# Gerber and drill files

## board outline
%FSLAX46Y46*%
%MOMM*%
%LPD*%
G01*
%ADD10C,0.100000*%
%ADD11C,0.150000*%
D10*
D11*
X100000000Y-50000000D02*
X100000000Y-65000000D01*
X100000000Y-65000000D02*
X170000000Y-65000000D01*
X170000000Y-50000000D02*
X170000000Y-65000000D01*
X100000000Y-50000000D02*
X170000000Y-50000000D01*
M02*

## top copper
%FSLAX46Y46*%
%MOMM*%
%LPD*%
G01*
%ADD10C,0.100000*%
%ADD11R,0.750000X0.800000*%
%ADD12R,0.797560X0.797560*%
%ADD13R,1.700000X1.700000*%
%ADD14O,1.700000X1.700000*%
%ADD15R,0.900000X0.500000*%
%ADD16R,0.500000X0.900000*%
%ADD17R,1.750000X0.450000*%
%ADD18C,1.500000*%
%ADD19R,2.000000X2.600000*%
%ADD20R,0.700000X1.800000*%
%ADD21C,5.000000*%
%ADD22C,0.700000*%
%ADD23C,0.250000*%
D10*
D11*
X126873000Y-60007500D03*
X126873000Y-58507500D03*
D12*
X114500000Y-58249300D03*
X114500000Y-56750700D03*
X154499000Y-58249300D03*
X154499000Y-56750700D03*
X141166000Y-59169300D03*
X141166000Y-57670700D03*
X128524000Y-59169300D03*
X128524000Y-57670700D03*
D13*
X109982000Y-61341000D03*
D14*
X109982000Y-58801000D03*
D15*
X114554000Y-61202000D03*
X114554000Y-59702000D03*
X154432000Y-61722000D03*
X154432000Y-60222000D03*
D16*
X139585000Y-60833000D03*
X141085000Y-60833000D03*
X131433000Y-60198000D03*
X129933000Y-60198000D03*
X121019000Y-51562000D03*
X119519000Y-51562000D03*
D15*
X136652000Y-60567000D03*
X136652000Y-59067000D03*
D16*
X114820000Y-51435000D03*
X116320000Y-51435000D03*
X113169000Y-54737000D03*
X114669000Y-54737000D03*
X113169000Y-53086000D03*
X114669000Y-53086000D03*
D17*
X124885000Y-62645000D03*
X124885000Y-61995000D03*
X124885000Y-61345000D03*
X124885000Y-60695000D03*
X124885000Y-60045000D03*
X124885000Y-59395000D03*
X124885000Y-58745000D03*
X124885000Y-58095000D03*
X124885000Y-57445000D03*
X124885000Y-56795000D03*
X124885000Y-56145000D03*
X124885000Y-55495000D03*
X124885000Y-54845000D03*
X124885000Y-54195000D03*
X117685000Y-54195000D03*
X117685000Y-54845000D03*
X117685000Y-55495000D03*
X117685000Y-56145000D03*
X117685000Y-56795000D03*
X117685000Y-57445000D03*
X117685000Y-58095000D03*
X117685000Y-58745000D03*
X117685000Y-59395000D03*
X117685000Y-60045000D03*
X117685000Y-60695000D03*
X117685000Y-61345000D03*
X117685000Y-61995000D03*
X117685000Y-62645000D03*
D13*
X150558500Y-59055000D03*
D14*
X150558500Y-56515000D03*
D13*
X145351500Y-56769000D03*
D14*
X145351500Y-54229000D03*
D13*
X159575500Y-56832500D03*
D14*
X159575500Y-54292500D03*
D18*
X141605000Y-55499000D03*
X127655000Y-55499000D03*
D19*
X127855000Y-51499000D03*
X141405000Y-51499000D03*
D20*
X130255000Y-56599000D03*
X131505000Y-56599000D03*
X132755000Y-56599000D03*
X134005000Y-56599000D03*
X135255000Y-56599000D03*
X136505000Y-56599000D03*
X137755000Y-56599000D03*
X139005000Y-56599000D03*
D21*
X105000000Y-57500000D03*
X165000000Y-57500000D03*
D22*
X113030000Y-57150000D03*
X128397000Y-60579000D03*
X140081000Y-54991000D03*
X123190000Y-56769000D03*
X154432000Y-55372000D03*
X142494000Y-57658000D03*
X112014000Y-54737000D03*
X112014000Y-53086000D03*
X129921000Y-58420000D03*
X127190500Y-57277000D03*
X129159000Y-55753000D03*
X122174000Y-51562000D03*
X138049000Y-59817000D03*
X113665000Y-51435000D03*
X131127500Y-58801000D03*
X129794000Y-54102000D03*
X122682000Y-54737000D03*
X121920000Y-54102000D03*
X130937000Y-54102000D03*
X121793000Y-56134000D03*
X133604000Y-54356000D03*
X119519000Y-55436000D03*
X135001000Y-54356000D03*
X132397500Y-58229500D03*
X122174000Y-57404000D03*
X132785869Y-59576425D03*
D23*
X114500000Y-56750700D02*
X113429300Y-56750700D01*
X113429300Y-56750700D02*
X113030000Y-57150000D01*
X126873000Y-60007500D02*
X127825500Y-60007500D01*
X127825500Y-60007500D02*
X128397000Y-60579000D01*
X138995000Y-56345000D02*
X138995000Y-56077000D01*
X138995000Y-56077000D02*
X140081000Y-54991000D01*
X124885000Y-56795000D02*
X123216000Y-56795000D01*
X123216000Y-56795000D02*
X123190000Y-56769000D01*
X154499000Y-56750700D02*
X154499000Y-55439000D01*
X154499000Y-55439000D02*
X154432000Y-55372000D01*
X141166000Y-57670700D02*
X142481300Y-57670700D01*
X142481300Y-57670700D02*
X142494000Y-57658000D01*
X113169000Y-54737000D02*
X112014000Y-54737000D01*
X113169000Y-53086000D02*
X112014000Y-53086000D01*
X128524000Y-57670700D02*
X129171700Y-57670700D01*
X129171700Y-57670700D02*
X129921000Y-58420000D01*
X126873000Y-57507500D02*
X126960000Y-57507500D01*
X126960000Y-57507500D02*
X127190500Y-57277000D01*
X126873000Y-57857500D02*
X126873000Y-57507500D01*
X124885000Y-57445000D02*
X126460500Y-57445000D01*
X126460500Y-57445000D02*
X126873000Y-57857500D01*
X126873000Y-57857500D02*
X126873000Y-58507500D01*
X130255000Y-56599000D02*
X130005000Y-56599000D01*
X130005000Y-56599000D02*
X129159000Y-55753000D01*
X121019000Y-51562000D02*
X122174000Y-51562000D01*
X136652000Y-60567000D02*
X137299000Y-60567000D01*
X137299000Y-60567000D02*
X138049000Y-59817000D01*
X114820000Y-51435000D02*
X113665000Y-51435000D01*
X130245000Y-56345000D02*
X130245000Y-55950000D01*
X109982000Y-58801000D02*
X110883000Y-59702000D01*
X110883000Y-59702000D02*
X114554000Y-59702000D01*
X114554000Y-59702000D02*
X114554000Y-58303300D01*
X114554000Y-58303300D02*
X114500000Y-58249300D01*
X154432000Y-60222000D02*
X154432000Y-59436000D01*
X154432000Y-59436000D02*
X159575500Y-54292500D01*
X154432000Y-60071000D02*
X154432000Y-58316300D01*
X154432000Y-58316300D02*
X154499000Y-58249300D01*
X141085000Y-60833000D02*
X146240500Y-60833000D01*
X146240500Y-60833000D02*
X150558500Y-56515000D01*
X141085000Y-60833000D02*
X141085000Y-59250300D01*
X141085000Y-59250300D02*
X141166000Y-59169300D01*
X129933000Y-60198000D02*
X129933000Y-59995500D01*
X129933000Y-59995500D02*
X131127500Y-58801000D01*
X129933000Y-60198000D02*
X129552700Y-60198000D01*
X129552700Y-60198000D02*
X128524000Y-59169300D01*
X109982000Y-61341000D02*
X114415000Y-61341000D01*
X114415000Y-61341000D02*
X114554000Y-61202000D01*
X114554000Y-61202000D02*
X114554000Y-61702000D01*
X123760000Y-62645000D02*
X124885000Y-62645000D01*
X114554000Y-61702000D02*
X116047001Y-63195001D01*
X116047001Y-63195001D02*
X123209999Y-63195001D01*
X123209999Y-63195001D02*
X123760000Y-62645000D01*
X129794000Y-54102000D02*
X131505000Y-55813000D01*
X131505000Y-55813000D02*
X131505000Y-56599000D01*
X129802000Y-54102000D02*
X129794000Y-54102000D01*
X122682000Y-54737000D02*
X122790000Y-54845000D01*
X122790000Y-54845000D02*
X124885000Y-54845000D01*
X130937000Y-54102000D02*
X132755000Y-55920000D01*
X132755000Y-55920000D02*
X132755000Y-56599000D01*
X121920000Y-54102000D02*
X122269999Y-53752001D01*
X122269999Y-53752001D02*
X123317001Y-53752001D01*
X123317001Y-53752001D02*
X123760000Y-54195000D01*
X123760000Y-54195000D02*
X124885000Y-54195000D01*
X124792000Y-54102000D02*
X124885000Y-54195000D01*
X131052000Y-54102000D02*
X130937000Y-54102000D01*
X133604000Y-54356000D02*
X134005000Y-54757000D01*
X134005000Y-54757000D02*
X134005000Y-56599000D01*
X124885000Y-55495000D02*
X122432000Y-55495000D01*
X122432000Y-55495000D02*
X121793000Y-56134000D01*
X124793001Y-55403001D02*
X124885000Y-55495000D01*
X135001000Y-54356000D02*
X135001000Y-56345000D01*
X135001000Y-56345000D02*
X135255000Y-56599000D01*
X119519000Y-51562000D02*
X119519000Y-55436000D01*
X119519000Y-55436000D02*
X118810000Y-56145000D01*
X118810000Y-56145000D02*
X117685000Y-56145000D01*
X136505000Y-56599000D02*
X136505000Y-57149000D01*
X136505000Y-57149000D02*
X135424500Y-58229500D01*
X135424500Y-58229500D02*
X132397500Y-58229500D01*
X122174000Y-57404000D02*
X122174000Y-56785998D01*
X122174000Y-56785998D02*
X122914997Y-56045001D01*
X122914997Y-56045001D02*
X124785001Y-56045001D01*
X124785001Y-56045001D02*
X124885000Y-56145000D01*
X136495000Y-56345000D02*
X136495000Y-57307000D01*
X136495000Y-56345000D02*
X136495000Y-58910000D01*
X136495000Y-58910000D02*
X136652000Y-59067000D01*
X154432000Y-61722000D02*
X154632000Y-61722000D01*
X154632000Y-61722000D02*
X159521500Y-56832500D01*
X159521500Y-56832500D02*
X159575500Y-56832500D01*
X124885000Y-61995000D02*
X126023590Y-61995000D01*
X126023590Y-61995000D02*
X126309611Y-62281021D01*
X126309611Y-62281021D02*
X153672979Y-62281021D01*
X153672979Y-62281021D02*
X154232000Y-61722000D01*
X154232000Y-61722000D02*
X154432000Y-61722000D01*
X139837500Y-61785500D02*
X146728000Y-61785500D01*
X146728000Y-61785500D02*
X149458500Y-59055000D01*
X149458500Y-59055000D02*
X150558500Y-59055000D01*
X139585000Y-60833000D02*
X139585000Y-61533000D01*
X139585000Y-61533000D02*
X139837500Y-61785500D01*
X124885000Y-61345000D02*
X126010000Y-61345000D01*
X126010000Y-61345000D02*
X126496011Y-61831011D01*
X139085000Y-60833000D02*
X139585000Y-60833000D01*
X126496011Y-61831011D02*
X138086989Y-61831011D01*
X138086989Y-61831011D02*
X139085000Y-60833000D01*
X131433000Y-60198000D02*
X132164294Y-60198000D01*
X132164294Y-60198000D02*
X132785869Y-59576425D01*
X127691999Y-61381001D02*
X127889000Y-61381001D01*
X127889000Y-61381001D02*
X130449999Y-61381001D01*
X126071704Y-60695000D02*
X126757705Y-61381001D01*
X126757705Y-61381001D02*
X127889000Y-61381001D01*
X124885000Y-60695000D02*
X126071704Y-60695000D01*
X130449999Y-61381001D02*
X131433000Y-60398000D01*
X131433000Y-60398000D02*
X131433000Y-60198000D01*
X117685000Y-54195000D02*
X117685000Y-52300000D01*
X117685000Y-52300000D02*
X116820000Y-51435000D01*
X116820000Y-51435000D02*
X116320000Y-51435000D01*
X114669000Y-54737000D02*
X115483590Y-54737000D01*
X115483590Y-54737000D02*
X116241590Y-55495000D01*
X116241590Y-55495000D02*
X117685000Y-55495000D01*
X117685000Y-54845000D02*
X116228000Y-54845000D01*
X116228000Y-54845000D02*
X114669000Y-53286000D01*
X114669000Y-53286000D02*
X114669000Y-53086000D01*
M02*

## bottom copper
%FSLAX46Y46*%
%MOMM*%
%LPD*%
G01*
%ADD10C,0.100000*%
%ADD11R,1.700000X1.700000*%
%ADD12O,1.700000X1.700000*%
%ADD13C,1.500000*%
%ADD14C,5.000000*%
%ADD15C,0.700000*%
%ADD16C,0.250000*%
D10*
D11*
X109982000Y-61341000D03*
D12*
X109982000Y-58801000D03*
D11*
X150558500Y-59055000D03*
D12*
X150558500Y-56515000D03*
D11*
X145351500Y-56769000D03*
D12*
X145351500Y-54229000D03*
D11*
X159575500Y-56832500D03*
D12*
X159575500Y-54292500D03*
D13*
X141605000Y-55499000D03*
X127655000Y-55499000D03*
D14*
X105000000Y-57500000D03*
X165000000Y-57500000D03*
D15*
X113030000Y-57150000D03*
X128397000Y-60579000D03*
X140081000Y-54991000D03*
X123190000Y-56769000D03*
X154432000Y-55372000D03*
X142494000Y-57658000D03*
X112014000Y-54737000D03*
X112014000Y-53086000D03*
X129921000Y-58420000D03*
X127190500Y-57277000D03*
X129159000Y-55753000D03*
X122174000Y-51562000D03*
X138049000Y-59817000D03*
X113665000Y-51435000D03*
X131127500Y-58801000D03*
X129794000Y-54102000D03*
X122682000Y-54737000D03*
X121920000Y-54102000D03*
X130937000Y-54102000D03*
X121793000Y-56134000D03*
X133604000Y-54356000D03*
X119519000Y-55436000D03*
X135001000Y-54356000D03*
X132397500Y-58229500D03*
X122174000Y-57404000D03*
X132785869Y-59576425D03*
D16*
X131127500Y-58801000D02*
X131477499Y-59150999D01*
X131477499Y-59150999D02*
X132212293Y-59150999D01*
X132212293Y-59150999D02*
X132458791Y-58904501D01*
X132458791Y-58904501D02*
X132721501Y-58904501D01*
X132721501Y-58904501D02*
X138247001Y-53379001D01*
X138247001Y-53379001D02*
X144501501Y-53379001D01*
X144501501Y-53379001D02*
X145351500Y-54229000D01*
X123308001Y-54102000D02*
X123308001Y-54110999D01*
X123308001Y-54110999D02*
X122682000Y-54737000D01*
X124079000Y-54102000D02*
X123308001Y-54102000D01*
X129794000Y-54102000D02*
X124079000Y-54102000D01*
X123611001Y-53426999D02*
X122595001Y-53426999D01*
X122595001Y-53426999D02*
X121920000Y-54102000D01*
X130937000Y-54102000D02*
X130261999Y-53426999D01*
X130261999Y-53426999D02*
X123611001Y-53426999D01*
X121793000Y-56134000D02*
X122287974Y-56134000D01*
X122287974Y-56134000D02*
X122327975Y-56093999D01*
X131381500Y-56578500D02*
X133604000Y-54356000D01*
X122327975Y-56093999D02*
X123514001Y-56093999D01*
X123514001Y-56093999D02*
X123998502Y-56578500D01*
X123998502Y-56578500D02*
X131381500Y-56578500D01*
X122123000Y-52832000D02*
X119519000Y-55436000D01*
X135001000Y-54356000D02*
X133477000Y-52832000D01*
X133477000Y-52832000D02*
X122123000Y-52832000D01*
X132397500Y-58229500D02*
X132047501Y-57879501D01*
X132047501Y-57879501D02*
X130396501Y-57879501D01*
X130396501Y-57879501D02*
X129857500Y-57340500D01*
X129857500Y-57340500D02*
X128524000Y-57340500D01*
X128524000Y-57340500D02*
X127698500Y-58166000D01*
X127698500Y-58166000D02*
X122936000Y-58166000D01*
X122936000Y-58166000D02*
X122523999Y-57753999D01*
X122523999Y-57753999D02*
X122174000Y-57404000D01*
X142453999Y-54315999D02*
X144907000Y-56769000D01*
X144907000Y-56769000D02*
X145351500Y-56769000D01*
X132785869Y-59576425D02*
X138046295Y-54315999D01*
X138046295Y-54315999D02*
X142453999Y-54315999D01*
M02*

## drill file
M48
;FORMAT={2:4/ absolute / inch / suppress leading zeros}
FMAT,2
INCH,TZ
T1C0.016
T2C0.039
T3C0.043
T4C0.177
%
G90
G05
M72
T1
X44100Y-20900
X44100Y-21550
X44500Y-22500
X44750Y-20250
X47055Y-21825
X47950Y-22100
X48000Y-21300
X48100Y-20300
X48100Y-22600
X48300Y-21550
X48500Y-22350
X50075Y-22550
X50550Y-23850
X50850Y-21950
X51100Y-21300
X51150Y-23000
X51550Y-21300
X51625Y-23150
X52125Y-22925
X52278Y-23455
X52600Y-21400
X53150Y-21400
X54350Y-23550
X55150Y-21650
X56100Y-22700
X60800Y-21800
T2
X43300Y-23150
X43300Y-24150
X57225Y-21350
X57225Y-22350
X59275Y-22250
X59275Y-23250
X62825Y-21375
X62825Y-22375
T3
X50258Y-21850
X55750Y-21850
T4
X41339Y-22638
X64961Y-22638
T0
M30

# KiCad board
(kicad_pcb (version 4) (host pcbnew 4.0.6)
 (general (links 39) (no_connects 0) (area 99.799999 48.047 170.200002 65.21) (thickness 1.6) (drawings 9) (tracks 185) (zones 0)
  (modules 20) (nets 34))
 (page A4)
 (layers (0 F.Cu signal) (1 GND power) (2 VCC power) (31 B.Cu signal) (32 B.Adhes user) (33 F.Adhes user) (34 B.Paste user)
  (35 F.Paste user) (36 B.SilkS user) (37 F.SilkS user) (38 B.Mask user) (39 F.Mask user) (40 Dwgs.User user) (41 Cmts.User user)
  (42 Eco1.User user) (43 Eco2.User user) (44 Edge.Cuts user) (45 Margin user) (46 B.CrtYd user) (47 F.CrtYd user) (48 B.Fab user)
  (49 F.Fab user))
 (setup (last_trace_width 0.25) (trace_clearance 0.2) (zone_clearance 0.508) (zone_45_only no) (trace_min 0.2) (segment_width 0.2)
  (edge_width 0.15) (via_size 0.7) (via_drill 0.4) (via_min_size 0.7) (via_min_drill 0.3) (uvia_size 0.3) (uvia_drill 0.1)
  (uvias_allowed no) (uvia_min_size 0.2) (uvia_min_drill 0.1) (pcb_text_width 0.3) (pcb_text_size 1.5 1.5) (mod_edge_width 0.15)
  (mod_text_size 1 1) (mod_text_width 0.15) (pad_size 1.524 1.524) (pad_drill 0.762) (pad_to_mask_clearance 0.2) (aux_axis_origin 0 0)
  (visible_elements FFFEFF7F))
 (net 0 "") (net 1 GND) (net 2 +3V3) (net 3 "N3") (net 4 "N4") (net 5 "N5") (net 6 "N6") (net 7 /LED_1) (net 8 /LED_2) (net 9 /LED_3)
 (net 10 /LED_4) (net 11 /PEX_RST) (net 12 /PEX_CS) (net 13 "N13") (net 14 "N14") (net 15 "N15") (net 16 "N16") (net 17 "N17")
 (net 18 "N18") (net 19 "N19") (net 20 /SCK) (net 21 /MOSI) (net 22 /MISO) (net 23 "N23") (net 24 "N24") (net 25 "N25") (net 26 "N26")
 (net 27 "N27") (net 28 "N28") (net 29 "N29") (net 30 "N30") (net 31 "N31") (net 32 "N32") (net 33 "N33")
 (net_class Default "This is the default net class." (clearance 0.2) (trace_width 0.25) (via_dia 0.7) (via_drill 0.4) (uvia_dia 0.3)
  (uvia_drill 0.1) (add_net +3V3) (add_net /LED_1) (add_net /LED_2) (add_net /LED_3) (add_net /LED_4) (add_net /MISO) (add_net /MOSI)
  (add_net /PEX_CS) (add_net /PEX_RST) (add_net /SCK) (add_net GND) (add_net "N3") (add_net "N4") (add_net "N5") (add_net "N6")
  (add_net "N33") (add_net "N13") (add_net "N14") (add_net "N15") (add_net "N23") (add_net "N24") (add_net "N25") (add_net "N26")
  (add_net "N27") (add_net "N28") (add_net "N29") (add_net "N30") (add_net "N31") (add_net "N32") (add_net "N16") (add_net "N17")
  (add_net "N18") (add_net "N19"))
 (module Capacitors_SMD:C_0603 (layer F.Cu) (at 126.873 59.2575 90)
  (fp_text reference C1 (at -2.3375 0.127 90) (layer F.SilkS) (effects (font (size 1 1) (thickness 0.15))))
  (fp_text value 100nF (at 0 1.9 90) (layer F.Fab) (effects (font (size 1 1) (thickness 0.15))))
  (pad 1 smd rect (at -0.75 0 90) (size 0.8 0.75) (layers F.Cu F.Paste F.Mask) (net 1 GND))
  (pad 2 smd rect (at 0.75 0 90) (size 0.8 0.75) (layers F.Cu F.Paste F.Mask) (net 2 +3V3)))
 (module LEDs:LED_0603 (layer F.Cu) (at 114.5 57.5 270)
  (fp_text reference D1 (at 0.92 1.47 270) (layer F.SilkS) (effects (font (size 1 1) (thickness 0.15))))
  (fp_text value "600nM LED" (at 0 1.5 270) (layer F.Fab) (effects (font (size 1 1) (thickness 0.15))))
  (pad 2 smd rect (at 0.7493 0 90) (size 0.79756 0.79756) (layers F.Cu F.Paste F.Mask) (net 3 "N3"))
  (pad 1 smd rect (at -0.7493 0 90) (size 0.79756 0.79756) (layers F.Cu F.Paste F.Mask) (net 1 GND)))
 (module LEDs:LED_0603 (layer F.Cu) (at 154.499 57.5 270)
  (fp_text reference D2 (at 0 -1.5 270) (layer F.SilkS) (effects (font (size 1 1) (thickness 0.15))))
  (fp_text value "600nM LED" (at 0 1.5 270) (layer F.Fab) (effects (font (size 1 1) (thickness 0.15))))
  (pad 2 smd rect (at 0.7493 0 90) (size 0.79756 0.79756) (layers F.Cu F.Paste F.Mask) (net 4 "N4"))
  (pad 1 smd rect (at -0.7493 0 90) (size 0.79756 0.79756) (layers F.Cu F.Paste F.Mask) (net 1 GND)))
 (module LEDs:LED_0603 (layer F.Cu) (at 141.166 58.42 270)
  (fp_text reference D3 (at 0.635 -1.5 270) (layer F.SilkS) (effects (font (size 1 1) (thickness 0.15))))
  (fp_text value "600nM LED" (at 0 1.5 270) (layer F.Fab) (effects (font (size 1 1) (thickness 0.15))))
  (pad 2 smd rect (at 0.7493 0 90) (size 0.79756 0.79756) (layers F.Cu F.Paste F.Mask) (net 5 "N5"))
  (pad 1 smd rect (at -0.7493 0 90) (size 0.79756 0.79756) (layers F.Cu F.Paste F.Mask) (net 1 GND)))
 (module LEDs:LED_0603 (layer F.Cu) (at 128.524 58.42 270)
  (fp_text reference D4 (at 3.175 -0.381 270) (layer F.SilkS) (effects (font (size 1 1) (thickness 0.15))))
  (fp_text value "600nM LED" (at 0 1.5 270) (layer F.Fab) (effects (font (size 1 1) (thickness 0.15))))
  (pad 2 smd rect (at 0.7493 0 90) (size 0.79756 0.79756) (layers F.Cu F.Paste F.Mask) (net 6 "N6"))
  (pad 1 smd rect (at -0.7493 0 90) (size 0.79756 0.79756) (layers F.Cu F.Paste F.Mask) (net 1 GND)))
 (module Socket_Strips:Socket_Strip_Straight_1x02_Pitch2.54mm (layer F.Cu) (at 109.982 61.341 180)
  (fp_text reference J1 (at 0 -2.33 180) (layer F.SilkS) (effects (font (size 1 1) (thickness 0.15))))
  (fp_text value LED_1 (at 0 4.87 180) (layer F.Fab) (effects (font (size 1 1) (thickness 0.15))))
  (pad 1 thru_hole rect (at 0 0 180) (size 1.7 1.7) (drill 1) (layers *.Cu *.Mask) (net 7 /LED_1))
  (pad 2 thru_hole oval (at 0 2.54 180) (size 1.7 1.7) (drill 1) (layers *.Cu *.Mask) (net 3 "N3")))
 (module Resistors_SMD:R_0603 (layer F.Cu) (at 114.554 60.452 90)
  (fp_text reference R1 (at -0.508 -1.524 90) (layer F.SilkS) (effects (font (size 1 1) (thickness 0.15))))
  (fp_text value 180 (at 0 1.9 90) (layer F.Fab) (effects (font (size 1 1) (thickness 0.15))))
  (pad 1 smd rect (at -0.75 0 90) (size 0.5 0.9) (layers F.Cu F.Paste F.Mask) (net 7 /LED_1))
  (pad 2 smd rect (at 0.75 0 90) (size 0.5 0.9) (layers F.Cu F.Paste F.Mask) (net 3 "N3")))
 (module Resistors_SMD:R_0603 (layer F.Cu) (at 154.432 60.972 90)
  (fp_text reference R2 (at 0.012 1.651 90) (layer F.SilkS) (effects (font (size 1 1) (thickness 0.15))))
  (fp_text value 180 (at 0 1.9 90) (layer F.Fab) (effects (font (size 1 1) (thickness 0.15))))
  (pad 1 smd rect (at -0.75 0 90) (size 0.5 0.9) (layers F.Cu F.Paste F.Mask) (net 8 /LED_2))
  (pad 2 smd rect (at 0.75 0 90) (size 0.5 0.9) (layers F.Cu F.Paste F.Mask) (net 4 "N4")))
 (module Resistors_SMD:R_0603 (layer F.Cu) (at 140.335 60.833)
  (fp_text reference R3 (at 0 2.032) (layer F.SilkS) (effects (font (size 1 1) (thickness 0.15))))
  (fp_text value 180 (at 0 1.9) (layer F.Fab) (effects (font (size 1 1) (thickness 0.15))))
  (pad 1 smd rect (at -0.75 0) (size 0.5 0.9) (layers F.Cu F.Paste F.Mask) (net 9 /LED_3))
  (pad 2 smd rect (at 0.75 0) (size 0.5 0.9) (layers F.Cu F.Paste F.Mask) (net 5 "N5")))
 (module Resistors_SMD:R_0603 (layer F.Cu) (at 130.683 60.198 180)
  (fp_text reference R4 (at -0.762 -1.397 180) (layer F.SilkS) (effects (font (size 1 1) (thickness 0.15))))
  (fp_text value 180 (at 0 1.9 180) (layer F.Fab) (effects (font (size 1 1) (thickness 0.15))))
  (pad 1 smd rect (at -0.75 0 180) (size 0.5 0.9) (layers F.Cu F.Paste F.Mask) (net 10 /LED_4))
  (pad 2 smd rect (at 0.75 0 180) (size 0.5 0.9) (layers F.Cu F.Paste F.Mask) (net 6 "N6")))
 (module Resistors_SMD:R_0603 (layer F.Cu) (at 120.269 51.562 180)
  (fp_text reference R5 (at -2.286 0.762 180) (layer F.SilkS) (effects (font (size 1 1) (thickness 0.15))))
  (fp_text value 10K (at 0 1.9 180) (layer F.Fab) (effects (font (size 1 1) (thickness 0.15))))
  (pad 1 smd rect (at -0.75 0 180) (size 0.5 0.9) (layers F.Cu F.Paste F.Mask) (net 2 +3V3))
  (pad 2 smd rect (at 0.75 0 180) (size 0.5 0.9) (layers F.Cu F.Paste F.Mask) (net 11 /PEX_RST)))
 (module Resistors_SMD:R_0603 (layer F.Cu) (at 136.652 59.817 90)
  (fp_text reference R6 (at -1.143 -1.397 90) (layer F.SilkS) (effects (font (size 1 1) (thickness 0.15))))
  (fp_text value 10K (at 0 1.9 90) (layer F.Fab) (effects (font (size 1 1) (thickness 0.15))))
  (pad 1 smd rect (at -0.75 0 90) (size 0.5 0.9) (layers F.Cu F.Paste F.Mask) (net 2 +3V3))
  (pad 2 smd rect (at 0.75 0 90) (size 0.5 0.9) (layers F.Cu F.Paste F.Mask) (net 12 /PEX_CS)))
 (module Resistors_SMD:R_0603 (layer F.Cu) (at 115.57 51.435)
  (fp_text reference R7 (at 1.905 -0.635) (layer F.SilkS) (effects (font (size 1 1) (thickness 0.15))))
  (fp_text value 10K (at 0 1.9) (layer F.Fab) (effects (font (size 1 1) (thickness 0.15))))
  (pad 1 smd rect (at -0.75 0) (size 0.5 0.9) (layers F.Cu F.Paste F.Mask) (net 2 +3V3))
  (pad 2 smd rect (at 0.75 0) (size 0.5 0.9) (layers F.Cu F.Paste F.Mask) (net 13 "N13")))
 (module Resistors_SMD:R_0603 (layer F.Cu) (at 113.919 54.737)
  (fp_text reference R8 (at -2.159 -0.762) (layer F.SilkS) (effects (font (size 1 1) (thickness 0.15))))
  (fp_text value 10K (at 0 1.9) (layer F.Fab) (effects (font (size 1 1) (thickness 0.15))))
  (pad 1 smd rect (at -0.75 0) (size 0.5 0.9) (layers F.Cu F.Paste F.Mask) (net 1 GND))
  (pad 2 smd rect (at 0.75 0) (size 0.5 0.9) (layers F.Cu F.Paste F.Mask) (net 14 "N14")))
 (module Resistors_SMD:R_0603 (layer F.Cu) (at 113.919 53.086)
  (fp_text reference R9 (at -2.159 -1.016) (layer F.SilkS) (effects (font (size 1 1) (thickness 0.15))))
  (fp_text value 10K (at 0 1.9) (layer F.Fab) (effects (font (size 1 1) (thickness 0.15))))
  (pad 1 smd rect (at -0.75 0) (size 0.5 0.9) (layers F.Cu F.Paste F.Mask) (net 1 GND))
  (pad 2 smd rect (at 0.75 0) (size 0.5 0.9) (layers F.Cu F.Paste F.Mask) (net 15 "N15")))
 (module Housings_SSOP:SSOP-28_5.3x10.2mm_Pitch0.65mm (layer F.Cu) (at 121.285 58.42 180)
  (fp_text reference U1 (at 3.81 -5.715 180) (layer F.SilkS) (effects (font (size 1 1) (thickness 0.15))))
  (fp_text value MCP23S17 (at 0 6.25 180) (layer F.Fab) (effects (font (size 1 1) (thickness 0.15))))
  (pad 1 smd rect (at -3.6 -4.225 180) (size 1.75 0.45) (layers F.Cu F.Paste F.Mask) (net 7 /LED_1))
  (pad 2 smd rect (at -3.6 -3.575 180) (size 1.75 0.45) (layers F.Cu F.Paste F.Mask) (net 8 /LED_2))
  (pad 3 smd rect (at -3.6 -2.925 180) (size 1.75 0.45) (layers F.Cu F.Paste F.Mask) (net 9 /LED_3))
  (pad 4 smd rect (at -3.6 -2.275 180) (size 1.75 0.45) (layers F.Cu F.Paste F.Mask) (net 10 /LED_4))
  (pad 5 smd rect (at -3.6 -1.625 180) (size 1.75 0.45) (layers F.Cu F.Paste F.Mask) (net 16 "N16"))
  (pad 6 smd rect (at -3.6 -0.975 180) (size 1.75 0.45) (layers F.Cu F.Paste F.Mask) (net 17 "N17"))
  (pad 7 smd rect (at -3.6 -0.325 180) (size 1.75 0.45) (layers F.Cu F.Paste F.Mask) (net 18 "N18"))
  (pad 8 smd rect (at -3.6 0.325 180) (size 1.75 0.45) (layers F.Cu F.Paste F.Mask) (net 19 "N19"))
  (pad 9 smd rect (at -3.6 0.975 180) (size 1.75 0.45) (layers F.Cu F.Paste F.Mask) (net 2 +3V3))
  (pad 10 smd rect (at -3.6 1.625 180) (size 1.75 0.45) (layers F.Cu F.Paste F.Mask) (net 1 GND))
  (pad 11 smd rect (at -3.6 2.275 180) (size 1.75 0.45) (layers F.Cu F.Paste F.Mask) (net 12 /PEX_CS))
  (pad 12 smd rect (at -3.6 2.925 180) (size 1.75 0.45) (layers F.Cu F.Paste F.Mask) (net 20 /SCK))
  (pad 13 smd rect (at -3.6 3.575 180) (size 1.75 0.45) (layers F.Cu F.Paste F.Mask) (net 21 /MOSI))
  (pad 14 smd rect (at -3.6 4.225 180) (size 1.75 0.45) (layers F.Cu F.Paste F.Mask) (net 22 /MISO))
  (pad 15 smd rect (at 3.6 4.225 180) (size 1.75 0.45) (layers F.Cu F.Paste F.Mask) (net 13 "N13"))
  (pad 16 smd rect (at 3.6 3.575 180) (size 1.75 0.45) (layers F.Cu F.Paste F.Mask) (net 15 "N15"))
  (pad 17 smd rect (at 3.6 2.925 180) (size 1.75 0.45) (layers F.Cu F.Paste F.Mask) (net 14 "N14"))
  (pad 18 smd rect (at 3.6 2.275 180) (size 1.75 0.45) (layers F.Cu F.Paste F.Mask) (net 11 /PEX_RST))
  (pad 19 smd rect (at 3.6 1.625 180) (size 1.75 0.45) (layers F.Cu F.Paste F.Mask) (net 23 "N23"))
  (pad 20 smd rect (at 3.6 0.975 180) (size 1.75 0.45) (layers F.Cu F.Paste F.Mask) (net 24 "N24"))
  (pad 21 smd rect (at 3.6 0.325 180) (size 1.75 0.45) (layers F.Cu F.Paste F.Mask) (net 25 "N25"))
  (pad 22 smd rect (at 3.6 -0.325 180) (size 1.75 0.45) (layers F.Cu F.Paste F.Mask) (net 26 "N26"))
  (pad 23 smd rect (at 3.6 -0.975 180) (size 1.75 0.45) (layers F.Cu F.Paste F.Mask) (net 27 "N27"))
  (pad 24 smd rect (at 3.6 -1.625 180) (size 1.75 0.45) (layers F.Cu F.Paste F.Mask) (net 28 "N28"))
  (pad 25 smd rect (at 3.6 -2.275 180) (size 1.75 0.45) (layers F.Cu F.Paste F.Mask) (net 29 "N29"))
  (pad 26 smd rect (at 3.6 -2.925 180) (size 1.75 0.45) (layers F.Cu F.Paste F.Mask) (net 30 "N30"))
  (pad 27 smd rect (at 3.6 -3.575 180) (size 1.75 0.45) (layers F.Cu F.Paste F.Mask) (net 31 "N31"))
  (pad 28 smd rect (at 3.6 -4.225 180) (size 1.75 0.45) (layers F.Cu F.Paste F.Mask) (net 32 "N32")))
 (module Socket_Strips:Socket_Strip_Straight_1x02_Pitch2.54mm (layer F.Cu) (at 150.5585 59.055 180)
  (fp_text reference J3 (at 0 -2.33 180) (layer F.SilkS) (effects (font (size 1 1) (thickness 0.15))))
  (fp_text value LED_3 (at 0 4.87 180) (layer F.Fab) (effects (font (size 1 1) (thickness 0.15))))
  (pad 1 thru_hole rect (at 0 0 180) (size 1.7 1.7) (drill 1) (layers *.Cu *.Mask) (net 9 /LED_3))
  (pad 2 thru_hole oval (at 0 2.54 180) (size 1.7 1.7) (drill 1) (layers *.Cu *.Mask) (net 5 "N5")))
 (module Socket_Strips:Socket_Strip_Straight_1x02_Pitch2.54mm (layer F.Cu) (at 145.3515 56.769 180)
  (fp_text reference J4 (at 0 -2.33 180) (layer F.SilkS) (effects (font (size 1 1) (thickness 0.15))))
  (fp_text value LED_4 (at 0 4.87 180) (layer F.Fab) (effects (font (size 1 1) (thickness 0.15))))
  (pad 1 thru_hole rect (at 0 0 180) (size 1.7 1.7) (drill 1) (layers *.Cu *.Mask) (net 10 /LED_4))
  (pad 2 thru_hole oval (at 0 2.54 180) (size 1.7 1.7) (drill 1) (layers *.Cu *.Mask) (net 6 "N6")))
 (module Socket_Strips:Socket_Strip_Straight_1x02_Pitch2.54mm (layer F.Cu) (at 159.5755 56.8325 180)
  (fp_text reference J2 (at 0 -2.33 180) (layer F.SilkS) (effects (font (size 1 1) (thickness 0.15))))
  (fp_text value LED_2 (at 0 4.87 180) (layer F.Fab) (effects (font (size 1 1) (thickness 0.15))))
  (pad 1 thru_hole rect (at 0 0 180) (size 1.7 1.7) (drill 1) (layers *.Cu *.Mask) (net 8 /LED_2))
  (pad 2 thru_hole oval (at 0 2.54 180) (size 1.7 1.7) (drill 1) (layers *.Cu *.Mask) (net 4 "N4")))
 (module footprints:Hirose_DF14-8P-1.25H (layer F.Cu) (at 134.63 55.499)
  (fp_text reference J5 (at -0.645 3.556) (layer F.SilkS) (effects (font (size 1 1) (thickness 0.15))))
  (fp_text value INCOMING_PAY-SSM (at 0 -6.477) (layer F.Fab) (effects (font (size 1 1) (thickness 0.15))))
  (pad ~ thru_hole circle (at 6.975 0) (size 1.5 1.5) (drill 1.1) (layers *.Cu *.Mask))
  (pad ~ thru_hole circle (at -6.975 0) (size 1.5 1.5) (drill 1.1) (layers *.Cu *.Mask))
  (pad ~ smd rect (at -6.775 -4) (size 2 2.6) (layers F.Cu F.Paste F.Mask))
  (pad ~ smd rect (at 6.775 -4) (size 2 2.6) (layers F.Cu F.Paste F.Mask))
  (pad 1 smd rect (at -4.375 1.1) (size 0.7 1.8) (layers F.Cu F.Paste F.Mask) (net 2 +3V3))
  (pad 2 smd rect (at -3.125 1.1) (size 0.7 1.8) (layers F.Cu F.Paste F.Mask) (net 21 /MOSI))
  (pad 3 smd rect (at -1.875 1.1) (size 0.7 1.8) (layers F.Cu F.Paste F.Mask) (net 22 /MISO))
  (pad 4 smd rect (at -0.625 1.1) (size 0.7 1.8) (layers F.Cu F.Paste F.Mask) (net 20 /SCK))
  (pad 5 smd rect (at 0.625 1.1) (size 0.7 1.8) (layers F.Cu F.Paste F.Mask) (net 11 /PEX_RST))
  (pad 6 smd rect (at 1.875 1.1) (size 0.7 1.8) (layers F.Cu F.Paste F.Mask) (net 12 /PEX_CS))
  (pad 7 smd rect (at 3.125 1.1) (size 0.7 1.8) (layers F.Cu F.Paste F.Mask) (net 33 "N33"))
  (pad 8 smd rect (at 4.375 1.1) (size 0.7 1.8) (layers F.Cu F.Paste F.Mask) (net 1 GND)))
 (gr_line (start 100 50) (end 100 65) (layer Edge.Cuts) (width 0.15))
 (gr_line (start 100 65) (end 170 65) (layer Edge.Cuts) (width 0.15))
 (gr_line (start 170 50) (end 170 65) (layer Edge.Cuts) (width 0.15))
 (gr_line (start 100 50) (end 170 50) (layer Edge.Cuts) (width 0.15))
 (via (at 105 57.5) (size 5) (drill 4.5) (layers F.Cu B.Cu) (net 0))
 (via (at 165 57.5) (size 5) (drill 4.5) (layers F.Cu B.Cu) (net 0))
 (segment (start 114.5 56.7507) (end 113.4293 56.7507) (width 0.25) (layer F.Cu) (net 1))
 (via (at 113.03 57.15) (size 0.7) (drill 0.4) (layers F.Cu B.Cu) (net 1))
 (segment (start 113.4293 56.7507) (end 113.03 57.15) (width 0.25) (layer F.Cu) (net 1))
 (segment (start 126.873 60.0075) (end 127.8255 60.0075) (width 0.25) (layer F.Cu) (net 1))
 (segment (start 127.8255 60.0075) (end 128.397 60.579) (width 0.25) (layer F.Cu) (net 1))
 (via (at 128.397 60.579) (size 0.7) (drill 0.4) (layers F.Cu B.Cu) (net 1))
 (segment (start 138.995 56.345) (end 138.995 56.077) (width 0.25) (layer F.Cu) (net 1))
 (segment (start 138.995 56.077) (end 140.081 54.991) (width 0.25) (layer F.Cu) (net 1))
 (via (at 140.081 54.991) (size 0.7) (drill 0.4) (layers F.Cu B.Cu) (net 1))
 (segment (start 124.885 56.795) (end 123.216 56.795) (width 0.25) (layer F.Cu) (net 1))
 (segment (start 123.216 56.795) (end 123.19 56.769) (width 0.25) (layer F.Cu) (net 1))
 (via (at 123.19 56.769) (size 0.7) (drill 0.4) (layers F.Cu B.Cu) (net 1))
 (segment (start 154.499 56.7507) (end 154.499 55.439) (width 0.25) (layer F.Cu) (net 1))
 (segment (start 154.499 55.439) (end 154.432 55.372) (width 0.25) (layer F.Cu) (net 1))
 (via (at 154.432 55.372) (size 0.7) (drill 0.4) (layers F.Cu B.Cu) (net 1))
 (segment (start 141.166 57.6707) (end 142.4813 57.6707) (width 0.25) (layer F.Cu) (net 1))
 (segment (start 142.4813 57.6707) (end 142.494 57.658) (width 0.25) (layer F.Cu) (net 1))
 (via (at 142.494 57.658) (size 0.7) (drill 0.4) (layers F.Cu B.Cu) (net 1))
 (segment (start 113.169 54.737) (end 112.014 54.737) (width 0.25) (layer F.Cu) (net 1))
 (via (at 112.014 54.737) (size 0.7) (drill 0.4) (layers F.Cu B.Cu) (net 1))
 (segment (start 113.169 53.086) (end 112.014 53.086) (width 0.25) (layer F.Cu) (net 1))
 (via (at 112.014 53.086) (size 0.7) (drill 0.4) (layers F.Cu B.Cu) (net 1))
 (segment (start 128.524 57.6707) (end 129.1717 57.6707) (width 0.25) (layer F.Cu) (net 1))
 (segment (start 129.1717 57.6707) (end 129.921 58.42) (width 0.25) (layer F.Cu) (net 1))
 (via (at 129.921 58.42) (size 0.7) (drill 0.4) (layers F.Cu B.Cu) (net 1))
 (segment (start 126.873 57.5075) (end 126.96 57.5075) (width 0.25) (layer F.Cu) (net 2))
 (segment (start 126.96 57.5075) (end 127.1905 57.277) (width 0.25) (layer F.Cu) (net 2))
 (via (at 127.1905 57.277) (size 0.7) (drill 0.4) (layers F.Cu B.Cu) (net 2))
 (segment (start 126.873 57.8575) (end 126.873 57.5075) (width 0.25) (layer F.Cu) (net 2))
 (segment (start 124.885 57.445) (end 126.4605 57.445) (width 0.25) (layer F.Cu) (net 2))
 (segment (start 126.4605 57.445) (end 126.873 57.8575) (width 0.25) (layer F.Cu) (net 2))
 (segment (start 126.873 57.8575) (end 126.873 58.5075) (width 0.25) (layer F.Cu) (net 2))
 (segment (start 130.255 56.599) (end 130.005 56.599) (width 0.25) (layer F.Cu) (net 2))
 (segment (start 130.005 56.599) (end 129.159 55.753) (width 0.25) (layer F.Cu) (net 2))
 (via (at 129.159 55.753) (size 0.7) (drill 0.4) (layers F.Cu B.Cu) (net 2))
 (segment (start 121.019 51.562) (end 122.174 51.562) (width 0.25) (layer F.Cu) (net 2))
 (via (at 122.174 51.562) (size 0.7) (drill 0.4) (layers F.Cu B.Cu) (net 2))
 (segment (start 136.652 60.567) (end 137.299 60.567) (width 0.25) (layer F.Cu) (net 2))
 (segment (start 137.299 60.567) (end 138.049 59.817) (width 0.25) (layer F.Cu) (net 2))
 (via (at 138.049 59.817) (size 0.7) (drill 0.4) (layers F.Cu B.Cu) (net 2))
 (segment (start 114.82 51.435) (end 113.665 51.435) (width 0.25) (layer F.Cu) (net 2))
 (via (at 113.665 51.435) (size 0.7) (drill 0.4) (layers F.Cu B.Cu) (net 2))
 (segment (start 130.245 56.345) (end 130.245 55.95) (width 0.25) (layer F.Cu) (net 2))
 (segment (start 109.982 58.801) (end 110.883 59.702) (width 0.25) (layer F.Cu) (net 3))
 (segment (start 110.883 59.702) (end 114.554 59.702) (width 0.25) (layer F.Cu) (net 3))
 (segment (start 114.554 59.702) (end 114.554 58.3033) (width 0.25) (layer F.Cu) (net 3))
 (segment (start 114.554 58.3033) (end 114.5 58.2493) (width 0.25) (layer F.Cu) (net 3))
 (segment (start 154.432 60.222) (end 154.432 59.436) (width 0.25) (layer F.Cu) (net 4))
 (segment (start 154.432 59.436) (end 159.5755 54.2925) (width 0.25) (layer F.Cu) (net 4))
 (segment (start 154.432 60.071) (end 154.432 58.3163) (width 0.25) (layer F.Cu) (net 4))
 (segment (start 154.432 58.3163) (end 154.499 58.2493) (width 0.25) (layer F.Cu) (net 4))
 (segment (start 141.085 60.833) (end 146.2405 60.833) (width 0.25) (layer F.Cu) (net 5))
 (segment (start 146.2405 60.833) (end 150.5585 56.515) (width 0.25) (layer F.Cu) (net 5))
 (segment (start 141.085 60.833) (end 141.085 59.2503) (width 0.25) (layer F.Cu) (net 5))
 (segment (start 141.085 59.2503) (end 141.166 59.1693) (width 0.25) (layer F.Cu) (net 5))
 (segment (start 131.1275 58.801) (end 131.477499 59.150999) (width 0.25) (layer B.Cu) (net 6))
 (segment (start 131.477499 59.150999) (end 132.212293 59.150999) (width 0.25) (layer B.Cu) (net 6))
 (segment (start 132.212293 59.150999) (end 132.458791 58.904501) (width 0.25) (layer B.Cu) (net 6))
 (segment (start 132.458791 58.904501) (end 132.721501 58.904501) (width 0.25) (layer B.Cu) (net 6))
 (segment (start 132.721501 58.904501) (end 138.247001 53.379001) (width 0.25) (layer B.Cu) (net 6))
 (segment (start 138.247001 53.379001) (end 144.501501 53.379001) (width 0.25) (layer B.Cu) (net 6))
 (segment (start 144.501501 53.379001) (end 145.3515 54.229) (width 0.25) (layer B.Cu) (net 6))
 (segment (start 129.933 60.198) (end 129.933 59.9955) (width 0.25) (layer F.Cu) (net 6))
 (segment (start 129.933 59.9955) (end 131.1275 58.801) (width 0.25) (layer F.Cu) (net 6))
 (via (at 131.1275 58.801) (size 0.7) (drill 0.4) (layers F.Cu B.Cu) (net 6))
 (segment (start 129.933 60.198) (end 129.5527 60.198) (width 0.25) (layer F.Cu) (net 6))
 (segment (start 129.5527 60.198) (end 128.524 59.1693) (width 0.25) (layer F.Cu) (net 6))
 (segment (start 109.982 61.341) (end 114.415 61.341) (width 0.25) (layer F.Cu) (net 7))
 (segment (start 114.415 61.341) (end 114.554 61.202) (width 0.25) (layer F.Cu) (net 7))
 (segment (start 114.554 61.202) (end 114.554 61.702) (width 0.25) (layer F.Cu) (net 7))
 (segment (start 123.76 62.645) (end 124.885 62.645) (width 0.25) (layer F.Cu) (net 7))
 (segment (start 114.554 61.702) (end 116.047001 63.195001) (width 0.25) (layer F.Cu) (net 7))
 (segment (start 116.047001 63.195001) (end 123.209999 63.195001) (width 0.25) (layer F.Cu) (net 7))
 (segment (start 123.209999 63.195001) (end 123.76 62.645) (width 0.25) (layer F.Cu) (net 7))
 (segment (start 129.794 54.102) (end 131.505 55.813) (width 0.25) (layer F.Cu) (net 21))
 (segment (start 131.505 55.813) (end 131.505 56.599) (width 0.25) (layer F.Cu) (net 21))
 (segment (start 129.802 54.102) (end 129.794 54.102) (width 0.25) (layer F.Cu) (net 21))
 (via (at 129.794 54.102) (size 0.7) (drill 0.4) (layers F.Cu B.Cu) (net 21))
 (segment (start 122.682 54.737) (end 122.79 54.845) (width 0.25) (layer F.Cu) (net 21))
 (segment (start 122.79 54.845) (end 124.885 54.845) (width 0.25) (layer F.Cu) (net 21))
 (segment (start 123.308001 54.102) (end 123.308001 54.110999) (width 0.25) (layer B.Cu) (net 21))
 (segment (start 123.308001 54.110999) (end 122.682 54.737) (width 0.25) (layer B.Cu) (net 21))
 (via (at 122.682 54.737) (size 0.7) (drill 0.4) (layers F.Cu B.Cu) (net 21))
 (segment (start 124.079 54.102) (end 123.308001 54.102) (width 0.25) (layer B.Cu) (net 21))
 (segment (start 129.794 54.102) (end 124.079 54.102) (width 0.25) (layer B.Cu) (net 21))
 (segment (start 130.937 54.102) (end 132.755 55.92) (width 0.25) (layer F.Cu) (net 22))
 (segment (start 132.755 55.92) (end 132.755 56.599) (width 0.25) (layer F.Cu) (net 22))
 (segment (start 121.92 54.102) (end 122.269999 53.752001) (width 0.25) (layer F.Cu) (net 22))
 (segment (start 122.269999 53.752001) (end 123.317001 53.752001) (width 0.25) (layer F.Cu) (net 22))
 (segment (start 123.317001 53.752001) (end 123.76 54.195) (width 0.25) (layer F.Cu) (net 22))
 (segment (start 123.76 54.195) (end 124.885 54.195) (width 0.25) (layer F.Cu) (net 22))
 (segment (start 123.611001 53.426999) (end 122.595001 53.426999) (width 0.25) (layer B.Cu) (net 22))
 (segment (start 122.595001 53.426999) (end 121.92 54.102) (width 0.25) (layer B.Cu) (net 22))
 (via (at 121.92 54.102) (size 0.7) (drill 0.4) (layers F.Cu B.Cu) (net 22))
 (segment (start 124.792 54.102) (end 124.885 54.195) (width 0.25) (layer F.Cu) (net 22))
 (segment (start 130.937 54.102) (end 130.261999 53.426999) (width 0.25) (layer B.Cu) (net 22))
 (segment (start 130.261999 53.426999) (end 123.611001 53.426999) (width 0.25) (layer B.Cu) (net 22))
 (segment (start 131.052 54.102) (end 130.937 54.102) (width 0.25) (layer F.Cu) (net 22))
 (via (at 130.937 54.102) (size 0.7) (drill 0.4) (layers F.Cu B.Cu) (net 22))
 (segment (start 121.793 56.134) (end 122.287974 56.134) (width 0.25) (layer B.Cu) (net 20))
 (segment (start 122.287974 56.134) (end 122.327975 56.093999) (width 0.25) (layer B.Cu) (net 20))
 (segment (start 131.3815 56.5785) (end 133.604 54.356) (width 0.25) (layer B.Cu) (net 20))
 (segment (start 122.327975 56.093999) (end 123.514001 56.093999) (width 0.25) (layer B.Cu) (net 20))
 (segment (start 123.514001 56.093999) (end 123.998502 56.5785) (width 0.25) (layer B.Cu) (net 20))
 (segment (start 123.998502 56.5785) (end 131.3815 56.5785) (width 0.25) (layer B.Cu) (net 20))
 (segment (start 133.604 54.356) (end 134.005 54.757) (width 0.25) (layer F.Cu) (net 20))
 (segment (start 134.005 54.757) (end 134.005 56.599) (width 0.25) (layer F.Cu) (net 20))
 (via (at 121.793 56.134) (size 0.7) (drill 0.4) (layers F.Cu B.Cu) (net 20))
 (segment (start 124.885 55.495) (end 122.432 55.495) (width 0.25) (layer F.Cu) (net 20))
 (segment (start 122.432 55.495) (end 121.793 56.134) (width 0.25) (layer F.Cu) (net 20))
 (segment (start 124.793001 55.403001) (end 124.885 55.495) (width 0.25) (layer F.Cu) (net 20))
 (via (at 133.604 54.356) (size 0.7) (drill 0.4) (layers F.Cu B.Cu) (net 20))
 (segment (start 135.001 54.356) (end 135.001 56.345) (width 0.25) (layer F.Cu) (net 11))
 (segment (start 135.001 56.345) (end 135.255 56.599) (width 0.25) (layer F.Cu) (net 11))
 (segment (start 122.123 52.832) (end 119.519 55.436) (width 0.25) (layer B.Cu) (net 11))
 (via (at 119.519 55.436) (size 0.7) (drill 0.4) (layers F.Cu B.Cu) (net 11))
 (segment (start 119.519 51.562) (end 119.519 55.436) (width 0.25) (layer F.Cu) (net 11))
 (segment (start 119.519 55.436) (end 118.81 56.145) (width 0.25) (layer F.Cu) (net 11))
 (segment (start 118.81 56.145) (end 117.685 56.145) (width 0.25) (layer F.Cu) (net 11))
 (segment (start 135.001 54.356) (end 133.477 52.832) (width 0.25) (layer B.Cu) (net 11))
 (segment (start 133.477 52.832) (end 122.123 52.832) (width 0.25) (layer B.Cu) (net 11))
 (via (at 135.001 54.356) (size 0.7) (drill 0.4) (layers F.Cu B.Cu) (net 11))
 (segment (start 132.3975 58.2295) (end 132.047501 57.879501) (width 0.25) (layer B.Cu) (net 12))
 (segment (start 132.047501 57.879501) (end 130.396501 57.879501) (width 0.25) (layer B.Cu) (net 12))
 (segment (start 130.396501 57.879501) (end 129.8575 57.3405) (width 0.25) (layer B.Cu) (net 12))
 (segment (start 129.8575 57.3405) (end 128.524 57.3405) (width 0.25) (layer B.Cu) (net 12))
 (segment (start 136.505 56.599) (end 136.505 57.149) (width 0.25) (layer F.Cu) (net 12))
 (segment (start 136.505 57.149) (end 135.4245 58.2295) (width 0.25) (layer F.Cu) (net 12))
 (segment (start 135.4245 58.2295) (end 132.3975 58.2295) (width 0.25) (layer F.Cu) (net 12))
 (via (at 132.3975 58.2295) (size 0.7) (drill 0.4) (layers F.Cu B.Cu) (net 12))
 (segment (start 128.524 57.3405) (end 127.6985 58.166) (width 0.25) (layer B.Cu) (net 12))
 (segment (start 127.6985 58.166) (end 122.936 58.166) (width 0.25) (layer B.Cu) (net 12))
 (segment (start 122.936 58.166) (end 122.523999 57.753999) (width 0.25) (layer B.Cu) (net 12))
 (segment (start 122.523999 57.753999) (end 122.174 57.404) (width 0.25) (layer B.Cu) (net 12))
 (via (at 122.174 57.404) (size 0.7) (drill 0.4) (layers F.Cu B.Cu) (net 12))
 (segment (start 122.174 57.404) (end 122.174 56.785998) (width 0.25) (layer F.Cu) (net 12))
 (segment (start 122.174 56.785998) (end 122.914997 56.045001) (width 0.25) (layer F.Cu) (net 12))
 (segment (start 122.914997 56.045001) (end 124.785001 56.045001) (width 0.25) (layer F.Cu) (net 12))
 (segment (start 124.785001 56.045001) (end 124.885 56.145) (width 0.25) (layer F.Cu) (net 12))
 (segment (start 136.495 56.345) (end 136.495 57.307) (width 0.25) (layer F.Cu) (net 12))
 (segment (start 136.495 56.345) (end 136.495 58.91) (width 0.25) (layer F.Cu) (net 12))
 (segment (start 136.495 58.91) (end 136.652 59.067) (width 0.25) (layer F.Cu) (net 12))
 (segment (start 154.432 61.722) (end 154.632 61.722) (width 0.25) (layer F.Cu) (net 8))
 (segment (start 154.632 61.722) (end 159.5215 56.8325) (width 0.25) (layer F.Cu) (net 8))
 (segment (start 159.5215 56.8325) (end 159.5755 56.8325) (width 0.25) (layer F.Cu) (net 8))
 (segment (start 124.885 61.995) (end 126.02359 61.995) (width 0.25) (layer F.Cu) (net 8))
 (segment (start 126.02359 61.995) (end 126.309611 62.281021) (width 0.25) (layer F.Cu) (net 8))
 (segment (start 126.309611 62.281021) (end 153.672979 62.281021) (width 0.25) (layer F.Cu) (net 8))
 (segment (start 153.672979 62.281021) (end 154.232 61.722) (width 0.25) (layer F.Cu) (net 8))
 (segment (start 154.232 61.722) (end 154.432 61.722) (width 0.25) (layer F.Cu) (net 8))
 (segment (start 139.8375 61.7855) (end 146.728 61.7855) (width 0.25) (layer F.Cu) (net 9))
 (segment (start 146.728 61.7855) (end 149.4585 59.055) (width 0.25) (layer F.Cu) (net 9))
 (segment (start 149.4585 59.055) (end 150.5585 59.055) (width 0.25) (layer F.Cu) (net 9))
 (segment (start 139.585 60.833) (end 139.585 61.533) (width 0.25) (layer F.Cu) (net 9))
 (segment (start 139.585 61.533) (end 139.8375 61.7855) (width 0.25) (layer F.Cu) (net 9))
 (segment (start 124.885 61.345) (end 126.01 61.345) (width 0.25) (layer F.Cu) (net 9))
 (segment (start 126.01 61.345) (end 126.496011 61.831011) (width 0.25) (layer F.Cu) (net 9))
 (segment (start 139.085 60.833) (end 139.585 60.833) (width 0.25) (layer F.Cu) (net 9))
 (segment (start 126.496011 61.831011) (end 138.086989 61.831011) (width 0.25) (layer F.Cu) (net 9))
 (segment (start 138.086989 61.831011) (end 139.085 60.833) (width 0.25) (layer F.Cu) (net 9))
 (segment (start 142.453999 54.315999) (end 144.907 56.769) (width 0.25) (layer B.Cu) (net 10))
 (segment (start 144.907 56.769) (end 145.3515 56.769) (width 0.25) (layer B.Cu) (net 10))
 (segment (start 132.785869 59.576425) (end 138.046295 54.315999) (width 0.25) (layer B.Cu) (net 10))
 (segment (start 138.046295 54.315999) (end 142.453999 54.315999) (width 0.25) (layer B.Cu) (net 10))
 (segment (start 131.433 60.198) (end 132.164294 60.198) (width 0.25) (layer F.Cu) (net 10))
 (segment (start 132.164294 60.198) (end 132.785869 59.576425) (width 0.25) (layer F.Cu) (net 10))
 (via (at 132.785869 59.576425) (size 0.7) (drill 0.4) (layers F.Cu B.Cu) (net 10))
 (segment (start 127.691999 61.381001) (end 127.889 61.381001) (width 0.25) (layer F.Cu) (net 10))
 (segment (start 127.889 61.381001) (end 130.449999 61.381001) (width 0.25) (layer F.Cu) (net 10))
 (segment (start 126.071704 60.695) (end 126.757705 61.381001) (width 0.25) (layer F.Cu) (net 10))
 (segment (start 126.757705 61.381001) (end 127.889 61.381001) (width 0.25) (layer F.Cu) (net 10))
 (segment (start 124.885 60.695) (end 126.071704 60.695) (width 0.25) (layer F.Cu) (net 10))
 (segment (start 130.449999 61.381001) (end 131.433 60.398) (width 0.25) (layer F.Cu) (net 10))
 (segment (start 131.433 60.398) (end 131.433 60.198) (width 0.25) (layer F.Cu) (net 10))
 (segment (start 117.685 54.195) (end 117.685 52.3) (width 0.25) (layer F.Cu) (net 13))
 (segment (start 117.685 52.3) (end 116.82 51.435) (width 0.25) (layer F.Cu) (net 13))
 (segment (start 116.82 51.435) (end 116.32 51.435) (width 0.25) (layer F.Cu) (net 13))
 (segment (start 114.669 54.737) (end 115.48359 54.737) (width 0.25) (layer F.Cu) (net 14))
 (segment (start 115.48359 54.737) (end 116.24159 55.495) (width 0.25) (layer F.Cu) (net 14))
 (segment (start 116.24159 55.495) (end 117.685 55.495) (width 0.25) (layer F.Cu) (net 14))
 (segment (start 117.685 54.845) (end 116.228 54.845) (width 0.25) (layer F.Cu) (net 15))
 (segment (start 116.228 54.845) (end 114.669 53.286) (width 0.25) (layer F.Cu) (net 15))
 (segment (start 114.669 53.286) (end 114.669 53.086) (width 0.25) (layer F.Cu) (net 15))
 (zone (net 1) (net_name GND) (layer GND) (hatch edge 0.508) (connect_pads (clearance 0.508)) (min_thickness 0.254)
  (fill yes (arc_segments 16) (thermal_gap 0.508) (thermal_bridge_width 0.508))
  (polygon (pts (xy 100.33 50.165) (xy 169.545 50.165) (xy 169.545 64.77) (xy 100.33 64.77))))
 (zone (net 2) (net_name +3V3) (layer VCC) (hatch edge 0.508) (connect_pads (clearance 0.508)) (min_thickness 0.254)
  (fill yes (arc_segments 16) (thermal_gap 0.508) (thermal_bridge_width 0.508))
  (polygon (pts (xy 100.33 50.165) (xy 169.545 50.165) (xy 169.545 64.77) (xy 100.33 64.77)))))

